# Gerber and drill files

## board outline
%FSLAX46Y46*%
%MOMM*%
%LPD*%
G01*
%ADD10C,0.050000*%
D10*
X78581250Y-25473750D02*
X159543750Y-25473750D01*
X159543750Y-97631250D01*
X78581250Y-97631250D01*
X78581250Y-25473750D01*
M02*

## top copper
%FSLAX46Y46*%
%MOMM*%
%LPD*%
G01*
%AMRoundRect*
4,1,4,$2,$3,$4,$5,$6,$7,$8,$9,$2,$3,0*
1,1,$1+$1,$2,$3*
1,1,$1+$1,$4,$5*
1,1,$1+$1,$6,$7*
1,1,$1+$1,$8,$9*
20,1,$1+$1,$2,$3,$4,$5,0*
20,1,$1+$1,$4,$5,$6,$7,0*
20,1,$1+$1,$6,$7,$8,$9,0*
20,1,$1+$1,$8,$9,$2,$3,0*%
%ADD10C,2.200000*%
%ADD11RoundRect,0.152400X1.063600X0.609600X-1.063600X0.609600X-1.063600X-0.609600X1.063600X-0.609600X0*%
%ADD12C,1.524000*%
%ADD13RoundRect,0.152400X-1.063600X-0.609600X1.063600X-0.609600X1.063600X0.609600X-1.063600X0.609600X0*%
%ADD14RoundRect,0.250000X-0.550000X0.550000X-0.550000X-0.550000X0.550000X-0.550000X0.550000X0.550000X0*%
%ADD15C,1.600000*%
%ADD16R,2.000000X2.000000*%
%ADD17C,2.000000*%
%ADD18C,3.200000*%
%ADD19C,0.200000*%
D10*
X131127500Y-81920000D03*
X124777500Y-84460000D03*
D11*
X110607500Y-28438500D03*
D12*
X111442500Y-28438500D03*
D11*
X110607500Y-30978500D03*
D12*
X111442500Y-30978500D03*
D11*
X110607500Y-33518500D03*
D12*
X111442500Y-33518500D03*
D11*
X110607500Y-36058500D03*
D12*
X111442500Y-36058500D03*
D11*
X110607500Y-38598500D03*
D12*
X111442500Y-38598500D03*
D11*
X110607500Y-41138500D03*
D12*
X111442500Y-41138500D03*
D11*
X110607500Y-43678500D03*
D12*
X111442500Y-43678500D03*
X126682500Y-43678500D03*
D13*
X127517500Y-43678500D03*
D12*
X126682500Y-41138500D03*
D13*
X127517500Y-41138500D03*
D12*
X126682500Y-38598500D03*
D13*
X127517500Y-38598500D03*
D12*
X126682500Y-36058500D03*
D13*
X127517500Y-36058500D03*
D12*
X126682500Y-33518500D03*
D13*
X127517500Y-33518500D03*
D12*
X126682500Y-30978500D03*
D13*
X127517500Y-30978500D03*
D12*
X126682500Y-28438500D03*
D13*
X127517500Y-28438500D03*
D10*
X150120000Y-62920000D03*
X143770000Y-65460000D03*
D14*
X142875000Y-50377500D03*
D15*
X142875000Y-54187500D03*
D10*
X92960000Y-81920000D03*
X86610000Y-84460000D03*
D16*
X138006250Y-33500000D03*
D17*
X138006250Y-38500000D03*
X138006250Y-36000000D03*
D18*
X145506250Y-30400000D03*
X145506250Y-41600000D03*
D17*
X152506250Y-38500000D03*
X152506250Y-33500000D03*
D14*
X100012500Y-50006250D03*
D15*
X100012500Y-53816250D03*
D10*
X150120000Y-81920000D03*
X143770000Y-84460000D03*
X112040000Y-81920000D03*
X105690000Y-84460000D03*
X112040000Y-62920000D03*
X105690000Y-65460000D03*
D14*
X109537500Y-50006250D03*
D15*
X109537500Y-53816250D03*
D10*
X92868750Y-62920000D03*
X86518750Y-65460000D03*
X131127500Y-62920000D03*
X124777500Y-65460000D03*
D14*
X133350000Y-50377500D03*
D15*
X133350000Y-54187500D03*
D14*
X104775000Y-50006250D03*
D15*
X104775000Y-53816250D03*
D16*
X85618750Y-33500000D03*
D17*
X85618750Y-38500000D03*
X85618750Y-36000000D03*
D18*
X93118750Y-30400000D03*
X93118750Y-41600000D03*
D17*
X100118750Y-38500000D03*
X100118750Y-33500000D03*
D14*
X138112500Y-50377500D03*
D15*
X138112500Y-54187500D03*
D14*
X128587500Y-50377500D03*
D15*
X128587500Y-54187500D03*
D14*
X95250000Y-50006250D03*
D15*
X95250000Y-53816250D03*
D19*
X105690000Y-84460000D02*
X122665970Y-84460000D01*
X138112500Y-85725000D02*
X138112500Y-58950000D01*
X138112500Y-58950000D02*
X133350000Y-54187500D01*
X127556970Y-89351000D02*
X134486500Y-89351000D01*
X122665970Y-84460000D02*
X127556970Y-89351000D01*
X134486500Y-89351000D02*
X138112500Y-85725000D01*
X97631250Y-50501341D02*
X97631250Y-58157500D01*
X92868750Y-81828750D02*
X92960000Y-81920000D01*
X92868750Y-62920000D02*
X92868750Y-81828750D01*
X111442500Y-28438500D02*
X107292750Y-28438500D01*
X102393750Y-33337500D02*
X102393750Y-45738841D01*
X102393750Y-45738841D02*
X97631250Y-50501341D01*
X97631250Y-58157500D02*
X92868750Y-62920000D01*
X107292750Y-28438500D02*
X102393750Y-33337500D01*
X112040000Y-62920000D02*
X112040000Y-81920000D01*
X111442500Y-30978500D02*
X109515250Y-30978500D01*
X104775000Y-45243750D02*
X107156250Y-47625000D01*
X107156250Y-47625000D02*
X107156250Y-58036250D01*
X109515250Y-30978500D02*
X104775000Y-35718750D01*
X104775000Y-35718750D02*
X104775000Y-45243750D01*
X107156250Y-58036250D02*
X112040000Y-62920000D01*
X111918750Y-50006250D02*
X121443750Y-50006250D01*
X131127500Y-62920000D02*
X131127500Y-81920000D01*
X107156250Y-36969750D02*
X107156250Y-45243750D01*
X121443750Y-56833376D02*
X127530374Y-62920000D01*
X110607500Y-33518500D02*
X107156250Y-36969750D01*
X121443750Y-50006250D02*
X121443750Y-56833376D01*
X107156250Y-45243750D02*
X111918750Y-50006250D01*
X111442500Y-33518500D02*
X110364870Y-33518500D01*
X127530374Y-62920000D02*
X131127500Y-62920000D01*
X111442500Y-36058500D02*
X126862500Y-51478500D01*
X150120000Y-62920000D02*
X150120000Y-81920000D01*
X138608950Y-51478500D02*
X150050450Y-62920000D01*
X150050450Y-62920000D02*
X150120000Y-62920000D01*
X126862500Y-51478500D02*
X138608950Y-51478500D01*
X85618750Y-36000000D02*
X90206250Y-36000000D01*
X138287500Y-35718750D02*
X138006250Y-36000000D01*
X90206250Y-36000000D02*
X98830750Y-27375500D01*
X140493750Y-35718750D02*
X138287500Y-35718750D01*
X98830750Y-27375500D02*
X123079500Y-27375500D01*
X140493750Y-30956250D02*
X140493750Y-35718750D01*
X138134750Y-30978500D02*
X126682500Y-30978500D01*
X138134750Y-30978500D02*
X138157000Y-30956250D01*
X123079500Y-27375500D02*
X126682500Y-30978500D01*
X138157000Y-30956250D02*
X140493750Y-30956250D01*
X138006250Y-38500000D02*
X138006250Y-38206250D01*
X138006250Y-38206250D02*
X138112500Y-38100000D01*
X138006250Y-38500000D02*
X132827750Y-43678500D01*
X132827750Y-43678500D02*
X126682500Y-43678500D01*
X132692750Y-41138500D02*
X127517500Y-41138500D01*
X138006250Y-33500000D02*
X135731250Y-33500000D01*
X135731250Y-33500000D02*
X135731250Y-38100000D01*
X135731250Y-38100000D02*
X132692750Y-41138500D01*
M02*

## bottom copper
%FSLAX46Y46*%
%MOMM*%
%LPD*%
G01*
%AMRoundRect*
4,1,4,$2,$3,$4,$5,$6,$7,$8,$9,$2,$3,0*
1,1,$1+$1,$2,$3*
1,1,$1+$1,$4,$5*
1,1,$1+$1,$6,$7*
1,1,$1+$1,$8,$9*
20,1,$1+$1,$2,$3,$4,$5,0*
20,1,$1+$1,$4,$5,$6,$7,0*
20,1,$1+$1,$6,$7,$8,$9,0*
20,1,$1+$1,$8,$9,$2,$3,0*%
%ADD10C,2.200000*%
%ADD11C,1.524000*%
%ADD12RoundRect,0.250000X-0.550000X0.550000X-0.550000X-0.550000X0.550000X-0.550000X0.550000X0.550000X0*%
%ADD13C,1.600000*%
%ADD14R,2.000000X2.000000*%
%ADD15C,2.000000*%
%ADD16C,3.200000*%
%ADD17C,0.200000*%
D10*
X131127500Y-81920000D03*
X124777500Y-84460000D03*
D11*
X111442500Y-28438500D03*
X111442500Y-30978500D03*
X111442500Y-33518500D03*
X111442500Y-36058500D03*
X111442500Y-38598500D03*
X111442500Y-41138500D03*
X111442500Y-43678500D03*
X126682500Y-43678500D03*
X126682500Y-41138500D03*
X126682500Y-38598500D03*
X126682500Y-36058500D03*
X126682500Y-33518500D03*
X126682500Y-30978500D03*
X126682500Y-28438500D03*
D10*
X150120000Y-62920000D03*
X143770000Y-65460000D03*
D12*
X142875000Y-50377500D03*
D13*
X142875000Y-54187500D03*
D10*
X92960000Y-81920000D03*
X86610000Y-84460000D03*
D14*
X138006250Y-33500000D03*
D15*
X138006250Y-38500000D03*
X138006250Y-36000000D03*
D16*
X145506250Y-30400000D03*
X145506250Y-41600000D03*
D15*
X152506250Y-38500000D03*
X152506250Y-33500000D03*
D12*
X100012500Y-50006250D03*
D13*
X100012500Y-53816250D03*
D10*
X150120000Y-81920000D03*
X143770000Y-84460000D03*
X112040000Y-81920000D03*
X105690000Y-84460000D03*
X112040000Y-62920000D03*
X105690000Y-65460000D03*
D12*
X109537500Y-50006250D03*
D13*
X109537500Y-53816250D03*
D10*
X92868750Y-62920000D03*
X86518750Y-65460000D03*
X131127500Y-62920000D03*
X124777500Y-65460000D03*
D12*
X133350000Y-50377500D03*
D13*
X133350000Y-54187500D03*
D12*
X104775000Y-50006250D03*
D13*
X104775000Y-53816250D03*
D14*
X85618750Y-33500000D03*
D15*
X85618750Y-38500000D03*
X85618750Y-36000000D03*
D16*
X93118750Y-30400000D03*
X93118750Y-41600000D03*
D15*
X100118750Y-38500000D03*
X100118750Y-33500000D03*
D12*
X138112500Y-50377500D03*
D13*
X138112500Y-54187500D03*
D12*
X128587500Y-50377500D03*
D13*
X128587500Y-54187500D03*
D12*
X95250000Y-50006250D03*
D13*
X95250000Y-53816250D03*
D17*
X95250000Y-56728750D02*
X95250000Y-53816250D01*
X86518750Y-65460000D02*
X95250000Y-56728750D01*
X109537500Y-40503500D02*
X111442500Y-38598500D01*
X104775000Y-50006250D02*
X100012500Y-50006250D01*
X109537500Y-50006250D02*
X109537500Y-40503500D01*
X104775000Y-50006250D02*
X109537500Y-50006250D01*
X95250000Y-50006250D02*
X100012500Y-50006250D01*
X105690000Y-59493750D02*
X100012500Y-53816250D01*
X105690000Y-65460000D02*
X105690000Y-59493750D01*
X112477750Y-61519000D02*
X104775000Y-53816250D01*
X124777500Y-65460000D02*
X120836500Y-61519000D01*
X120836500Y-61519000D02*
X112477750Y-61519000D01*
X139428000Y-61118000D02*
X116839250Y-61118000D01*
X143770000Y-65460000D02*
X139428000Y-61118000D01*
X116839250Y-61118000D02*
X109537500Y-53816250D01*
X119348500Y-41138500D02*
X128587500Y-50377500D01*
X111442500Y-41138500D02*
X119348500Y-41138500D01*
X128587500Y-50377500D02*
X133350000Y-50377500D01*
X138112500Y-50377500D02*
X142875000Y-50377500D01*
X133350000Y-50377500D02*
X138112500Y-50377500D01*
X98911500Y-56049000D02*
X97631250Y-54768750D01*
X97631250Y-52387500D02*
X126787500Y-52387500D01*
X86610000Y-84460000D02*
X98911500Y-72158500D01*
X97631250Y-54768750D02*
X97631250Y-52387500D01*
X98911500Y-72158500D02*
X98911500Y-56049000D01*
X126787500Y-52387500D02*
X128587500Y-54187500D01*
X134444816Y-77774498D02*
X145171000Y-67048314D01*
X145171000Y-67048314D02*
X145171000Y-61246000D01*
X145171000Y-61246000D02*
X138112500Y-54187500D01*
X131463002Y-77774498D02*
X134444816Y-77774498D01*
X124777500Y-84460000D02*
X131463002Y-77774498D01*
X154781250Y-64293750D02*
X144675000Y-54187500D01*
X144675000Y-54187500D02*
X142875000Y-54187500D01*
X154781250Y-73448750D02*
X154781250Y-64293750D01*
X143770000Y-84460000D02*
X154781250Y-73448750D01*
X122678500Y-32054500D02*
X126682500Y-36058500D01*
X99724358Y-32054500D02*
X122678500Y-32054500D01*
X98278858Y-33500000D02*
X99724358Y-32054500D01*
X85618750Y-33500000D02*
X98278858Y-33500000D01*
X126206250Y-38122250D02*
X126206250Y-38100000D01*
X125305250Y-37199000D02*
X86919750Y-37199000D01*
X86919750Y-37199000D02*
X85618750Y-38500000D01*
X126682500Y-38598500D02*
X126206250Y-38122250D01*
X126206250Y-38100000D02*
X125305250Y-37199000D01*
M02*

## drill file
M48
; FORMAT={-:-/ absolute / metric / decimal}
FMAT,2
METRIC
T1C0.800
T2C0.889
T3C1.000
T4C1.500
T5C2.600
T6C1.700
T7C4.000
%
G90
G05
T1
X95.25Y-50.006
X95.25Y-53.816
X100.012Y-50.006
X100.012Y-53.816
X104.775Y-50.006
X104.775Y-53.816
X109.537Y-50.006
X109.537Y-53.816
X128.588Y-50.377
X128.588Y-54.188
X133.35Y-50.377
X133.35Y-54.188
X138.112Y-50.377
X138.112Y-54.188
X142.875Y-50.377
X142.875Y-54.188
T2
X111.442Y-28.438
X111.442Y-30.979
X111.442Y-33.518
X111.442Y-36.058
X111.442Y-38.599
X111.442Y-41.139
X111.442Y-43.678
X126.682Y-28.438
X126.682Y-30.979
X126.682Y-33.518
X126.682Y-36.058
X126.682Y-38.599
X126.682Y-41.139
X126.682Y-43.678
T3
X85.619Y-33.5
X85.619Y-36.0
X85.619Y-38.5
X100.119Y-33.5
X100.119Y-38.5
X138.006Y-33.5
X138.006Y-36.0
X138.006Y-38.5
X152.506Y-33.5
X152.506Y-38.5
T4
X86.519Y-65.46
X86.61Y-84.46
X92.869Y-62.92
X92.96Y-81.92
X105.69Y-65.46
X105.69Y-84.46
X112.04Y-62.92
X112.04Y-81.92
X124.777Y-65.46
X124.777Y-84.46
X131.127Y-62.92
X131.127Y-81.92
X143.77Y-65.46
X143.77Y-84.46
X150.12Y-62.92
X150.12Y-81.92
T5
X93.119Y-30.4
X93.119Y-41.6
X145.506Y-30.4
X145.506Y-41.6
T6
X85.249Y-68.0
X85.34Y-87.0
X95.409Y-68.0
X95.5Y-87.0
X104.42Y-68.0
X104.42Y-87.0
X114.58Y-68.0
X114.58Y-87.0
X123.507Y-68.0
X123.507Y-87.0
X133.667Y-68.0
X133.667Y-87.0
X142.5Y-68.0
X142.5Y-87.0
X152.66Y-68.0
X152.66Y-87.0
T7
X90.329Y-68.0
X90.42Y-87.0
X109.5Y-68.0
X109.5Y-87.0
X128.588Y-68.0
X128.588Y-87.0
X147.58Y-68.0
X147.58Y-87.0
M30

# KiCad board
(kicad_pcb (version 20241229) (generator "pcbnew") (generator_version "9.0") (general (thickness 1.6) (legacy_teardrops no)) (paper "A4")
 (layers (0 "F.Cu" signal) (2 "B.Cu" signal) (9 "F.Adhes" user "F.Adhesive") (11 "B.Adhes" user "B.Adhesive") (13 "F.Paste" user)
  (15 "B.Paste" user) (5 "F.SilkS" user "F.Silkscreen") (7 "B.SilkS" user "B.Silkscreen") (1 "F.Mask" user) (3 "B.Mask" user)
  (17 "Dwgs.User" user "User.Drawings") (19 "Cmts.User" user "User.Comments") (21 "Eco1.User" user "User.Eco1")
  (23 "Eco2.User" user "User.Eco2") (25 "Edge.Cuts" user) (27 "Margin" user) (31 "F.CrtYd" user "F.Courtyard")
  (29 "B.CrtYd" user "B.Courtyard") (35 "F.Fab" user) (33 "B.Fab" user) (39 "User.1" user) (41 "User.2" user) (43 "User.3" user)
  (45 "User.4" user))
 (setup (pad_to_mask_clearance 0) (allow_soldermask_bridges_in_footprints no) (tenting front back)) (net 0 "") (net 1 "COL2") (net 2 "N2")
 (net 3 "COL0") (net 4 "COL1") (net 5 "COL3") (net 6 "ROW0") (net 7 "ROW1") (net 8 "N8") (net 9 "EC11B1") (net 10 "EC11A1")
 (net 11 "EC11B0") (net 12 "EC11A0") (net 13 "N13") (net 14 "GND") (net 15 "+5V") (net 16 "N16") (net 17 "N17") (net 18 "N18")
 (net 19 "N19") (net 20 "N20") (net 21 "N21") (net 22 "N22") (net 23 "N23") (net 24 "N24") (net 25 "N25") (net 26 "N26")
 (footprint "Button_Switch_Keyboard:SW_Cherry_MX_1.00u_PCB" (layer "F.Cu") (at 131.1275 81.92)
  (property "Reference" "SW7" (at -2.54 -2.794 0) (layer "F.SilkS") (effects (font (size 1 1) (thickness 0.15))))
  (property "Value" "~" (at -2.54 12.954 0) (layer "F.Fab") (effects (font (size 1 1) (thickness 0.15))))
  (pad "" np_thru_hole circle (at -7.62 5.08) (size 1.7 1.7) (drill 1.7) (layers "*.Cu" "*.Mask"))
  (pad "" np_thru_hole circle (at -2.54 5.08) (size 4 4) (drill 4) (layers "*.Cu" "*.Mask"))
  (pad "" np_thru_hole circle (at 2.54 5.08) (size 1.7 1.7) (drill 1.7) (layers "*.Cu" "*.Mask"))
  (pad "1" thru_hole circle (at 0 0) (size 2.2 2.2) (drill 1.5) (layers "*.Cu" "*.Mask") (remove_unused_layers no) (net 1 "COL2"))
  (pad "2" thru_hole circle (at -6.35 2.54) (size 2.2 2.2) (drill 1.5) (layers "*.Cu" "*.Mask") (remove_unused_layers no) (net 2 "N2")))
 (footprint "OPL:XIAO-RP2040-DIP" (layer "F.Cu") (at 119.0625 36.0585)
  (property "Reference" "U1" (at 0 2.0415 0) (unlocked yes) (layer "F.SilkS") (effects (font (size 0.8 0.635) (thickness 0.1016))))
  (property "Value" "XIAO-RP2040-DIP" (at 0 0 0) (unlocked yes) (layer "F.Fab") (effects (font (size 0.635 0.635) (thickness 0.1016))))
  (pad "1" smd roundrect (at -8.455 -7.62 180) (size 2.432 1.524) (layers "F.Cu" "F.Mask") (roundrect_rratio 0.1) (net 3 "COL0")
   (thermal_bridge_angle 45))
  (pad "1" thru_hole circle (at -7.62 -7.62 180) (size 1.524 1.524) (drill 0.889) (layers "*.Cu" "*.Mask") (remove_unused_layers no)
   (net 3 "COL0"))
  (pad "2" smd roundrect (at -8.455 -5.08 180) (size 2.432 1.524) (layers "F.Cu" "F.Mask") (roundrect_rratio 0.1) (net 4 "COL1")
   (thermal_bridge_angle 45))
  (pad "2" thru_hole circle (at -7.62 -5.08 180) (size 1.524 1.524) (drill 0.889) (layers "*.Cu" "*.Mask") (remove_unused_layers no)
   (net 4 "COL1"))
  (pad "3" smd roundrect (at -8.455 -2.54 180) (size 2.432 1.524) (layers "F.Cu" "F.Mask") (roundrect_rratio 0.1) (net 1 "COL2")
   (thermal_bridge_angle 45))
  (pad "3" thru_hole circle (at -7.62 -2.54 180) (size 1.524 1.524) (drill 0.889) (layers "*.Cu" "*.Mask") (remove_unused_layers no)
   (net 1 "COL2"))
  (pad "4" smd roundrect (at -8.455 0 180) (size 2.432 1.524) (layers "F.Cu" "F.Mask") (roundrect_rratio 0.1) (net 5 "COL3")
   (thermal_bridge_angle 45))
  (pad "4" thru_hole circle (at -7.62 0 180) (size 1.524 1.524) (drill 0.889) (layers "*.Cu" "*.Mask") (remove_unused_layers no)
   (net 5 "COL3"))
  (pad "5" smd roundrect (at -8.455 2.54 180) (size 2.432 1.524) (layers "F.Cu" "F.Mask") (roundrect_rratio 0.1) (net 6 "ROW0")
   (thermal_bridge_angle 45))
  (pad "5" thru_hole circle (at -7.62 2.54 180) (size 1.524 1.524) (drill 0.889) (layers "*.Cu" "*.Mask") (remove_unused_layers no)
   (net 6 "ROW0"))
  (pad "6" smd roundrect (at -8.455 5.08 180) (size 2.432 1.524) (layers "F.Cu" "F.Mask") (roundrect_rratio 0.1) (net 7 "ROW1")
   (thermal_bridge_angle 45))
  (pad "6" thru_hole circle (at -7.62 5.08 180) (size 1.524 1.524) (drill 0.889) (layers "*.Cu" "*.Mask") (remove_unused_layers no)
   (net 7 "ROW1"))
  (pad "7" smd roundrect (at -8.455 7.62 180) (size 2.432 1.524) (layers "F.Cu" "F.Mask") (roundrect_rratio 0.1) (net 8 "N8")
   (thermal_bridge_angle 45))
  (pad "7" thru_hole circle (at -7.62 7.62 180) (size 1.524 1.524) (drill 0.889) (layers "*.Cu" "*.Mask") (remove_unused_layers no)
   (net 8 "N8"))
  (pad "8" thru_hole circle (at 7.62 7.62) (size 1.524 1.524) (drill 0.889) (layers "*.Cu" "*.Mask") (remove_unused_layers no)
   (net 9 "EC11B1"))
  (pad "8" smd roundrect (at 8.455 7.62) (size 2.432 1.524) (layers "F.Cu" "F.Mask") (roundrect_rratio 0.1) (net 9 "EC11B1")
   (thermal_bridge_angle 45))
  (pad "9" thru_hole circle (at 7.62 5.08) (size 1.524 1.524) (drill 0.889) (layers "*.Cu" "*.Mask") (remove_unused_layers no)
   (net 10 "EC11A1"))
  (pad "9" smd roundrect (at 8.455 5.08) (size 2.432 1.524) (layers "F.Cu" "F.Mask") (roundrect_rratio 0.1) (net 10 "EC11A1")
   (thermal_bridge_angle 45))
  (pad "10" thru_hole circle (at 7.62 2.54) (size 1.524 1.524) (drill 0.889) (layers "*.Cu" "*.Mask") (remove_unused_layers no)
   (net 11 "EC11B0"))
  (pad "10" smd roundrect (at 8.455 2.54) (size 2.432 1.524) (layers "F.Cu" "F.Mask") (roundrect_rratio 0.1) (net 11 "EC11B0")
   (thermal_bridge_angle 45))
  (pad "11" thru_hole circle (at 7.62 0) (size 1.524 1.524) (drill 0.889) (layers "*.Cu" "*.Mask") (remove_unused_layers no)
   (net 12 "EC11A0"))
  (pad "11" smd roundrect (at 8.455 0) (size 2.432 1.524) (layers "F.Cu" "F.Mask") (roundrect_rratio 0.1) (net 12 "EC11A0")
   (thermal_bridge_angle 45))
  (pad "12" thru_hole circle (at 7.62 -2.54) (size 1.524 1.524) (drill 0.889) (layers "*.Cu" "*.Mask") (remove_unused_layers no)
   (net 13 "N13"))
  (pad "12" smd roundrect (at 8.455 -2.54) (size 2.432 1.524) (layers "F.Cu" "F.Mask") (roundrect_rratio 0.1) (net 13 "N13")
   (thermal_bridge_angle 45))
  (pad "13" thru_hole circle (at 7.62 -5.08) (size 1.524 1.524) (drill 0.889) (layers "*.Cu" "*.Mask") (remove_unused_layers no)
   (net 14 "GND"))
  (pad "13" smd roundrect (at 8.455 -5.08) (size 2.432 1.524) (layers "F.Cu" "F.Mask") (roundrect_rratio 0.1) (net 14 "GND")
   (thermal_bridge_angle 45))
  (pad "14" thru_hole circle (at 7.62 -7.62) (size 1.524 1.524) (drill 0.889) (layers "*.Cu" "*.Mask") (remove_unused_layers no)
   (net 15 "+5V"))
  (pad "14" smd roundrect (at 8.455 -7.62) (size 2.432 1.524) (layers "F.Cu" "F.Mask") (roundrect_rratio 0.1) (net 15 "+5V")
   (thermal_bridge_angle 45)))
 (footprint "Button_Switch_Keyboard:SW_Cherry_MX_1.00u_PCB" (layer "F.Cu") (at 150.12 62.92)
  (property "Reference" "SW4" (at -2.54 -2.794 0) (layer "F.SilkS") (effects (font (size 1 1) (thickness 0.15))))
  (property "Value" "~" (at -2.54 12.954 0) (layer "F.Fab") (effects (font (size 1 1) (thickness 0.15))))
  (pad "" np_thru_hole circle (at -7.62 5.08) (size 1.7 1.7) (drill 1.7) (layers "*.Cu" "*.Mask"))
  (pad "" np_thru_hole circle (at -2.54 5.08) (size 4 4) (drill 4) (layers "*.Cu" "*.Mask"))
  (pad "" np_thru_hole circle (at 2.54 5.08) (size 1.7 1.7) (drill 1.7) (layers "*.Cu" "*.Mask"))
  (pad "1" thru_hole circle (at 0 0) (size 2.2 2.2) (drill 1.5) (layers "*.Cu" "*.Mask") (remove_unused_layers no) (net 5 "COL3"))
  (pad "2" thru_hole circle (at -6.35 2.54) (size 2.2 2.2) (drill 1.5) (layers "*.Cu" "*.Mask") (remove_unused_layers no) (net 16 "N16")))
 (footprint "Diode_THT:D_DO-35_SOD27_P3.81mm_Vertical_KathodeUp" (layer "F.Cu") (at 142.875 50.3775 -90)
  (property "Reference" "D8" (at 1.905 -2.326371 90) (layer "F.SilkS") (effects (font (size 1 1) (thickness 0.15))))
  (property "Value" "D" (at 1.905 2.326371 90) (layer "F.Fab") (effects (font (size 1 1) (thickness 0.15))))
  (pad "1" thru_hole roundrect (at 0 0 270) (size 1.6 1.6) (drill 0.8) (layers "*.Cu" "*.Mask") (remove_unused_layers no)
   (roundrect_rratio 0.15625) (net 7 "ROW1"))
  (pad "2" thru_hole circle (at 3.81 0 270) (size 1.6 1.6) (drill 0.8) (layers "*.Cu" "*.Mask") (remove_unused_layers no) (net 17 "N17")))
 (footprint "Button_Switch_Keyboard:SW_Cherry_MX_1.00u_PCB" (layer "F.Cu") (at 92.96 81.92)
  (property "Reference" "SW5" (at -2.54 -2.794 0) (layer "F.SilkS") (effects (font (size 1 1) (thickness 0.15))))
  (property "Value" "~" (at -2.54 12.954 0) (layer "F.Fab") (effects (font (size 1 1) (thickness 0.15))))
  (pad "" np_thru_hole circle (at -7.62 5.08) (size 1.7 1.7) (drill 1.7) (layers "*.Cu" "*.Mask"))
  (pad "" np_thru_hole circle (at -2.54 5.08) (size 4 4) (drill 4) (layers "*.Cu" "*.Mask"))
  (pad "" np_thru_hole circle (at 2.54 5.08) (size 1.7 1.7) (drill 1.7) (layers "*.Cu" "*.Mask"))
  (pad "1" thru_hole circle (at 0 0) (size 2.2 2.2) (drill 1.5) (layers "*.Cu" "*.Mask") (remove_unused_layers no) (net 3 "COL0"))
  (pad "2" thru_hole circle (at -6.35 2.54) (size 2.2 2.2) (drill 1.5) (layers "*.Cu" "*.Mask") (remove_unused_layers no) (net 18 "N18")))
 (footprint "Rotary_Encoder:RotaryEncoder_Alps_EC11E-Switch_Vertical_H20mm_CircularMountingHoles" (layer "F.Cu") (at 138.00625 33.5)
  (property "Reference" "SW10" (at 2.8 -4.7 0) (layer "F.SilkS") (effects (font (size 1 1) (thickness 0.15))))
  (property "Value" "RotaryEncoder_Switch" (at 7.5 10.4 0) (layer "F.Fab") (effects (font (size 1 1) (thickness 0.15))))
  (pad "A" thru_hole rect (at 0 0) (size 2 2) (drill 1) (layers "*.Cu" "*.Mask") (remove_unused_layers no) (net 10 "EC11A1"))
  (pad "B" thru_hole circle (at 0 5) (size 2 2) (drill 1) (layers "*.Cu" "*.Mask") (remove_unused_layers no) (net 9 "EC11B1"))
  (pad "C" thru_hole circle (at 0 2.5) (size 2 2) (drill 1) (layers "*.Cu" "*.Mask") (remove_unused_layers no) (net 14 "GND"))
  (pad "MP" thru_hole circle (at 7.5 -3.1) (size 3.2 3.2) (drill 2.6) (layers "*.Cu" "*.Mask") (remove_unused_layers no))
  (pad "MP" thru_hole circle (at 7.5 8.1) (size 3.2 3.2) (drill 2.6) (layers "*.Cu" "*.Mask") (remove_unused_layers no))
  (pad "S1" thru_hole circle (at 14.5 5) (size 2 2) (drill 1) (layers "*.Cu" "*.Mask") (remove_unused_layers no) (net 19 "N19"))
  (pad "S2" thru_hole circle (at 14.5 0) (size 2 2) (drill 1) (layers "*.Cu" "*.Mask") (remove_unused_layers no) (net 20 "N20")))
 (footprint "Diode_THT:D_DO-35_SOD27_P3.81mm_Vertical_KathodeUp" (layer "F.Cu") (at 100.0125 50.00625 -90)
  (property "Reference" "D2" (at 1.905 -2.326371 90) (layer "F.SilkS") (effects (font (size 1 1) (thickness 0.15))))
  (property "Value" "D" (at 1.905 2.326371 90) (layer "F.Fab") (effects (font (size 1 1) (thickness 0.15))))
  (pad "1" thru_hole roundrect (at 0 0 270) (size 1.6 1.6) (drill 0.8) (layers "*.Cu" "*.Mask") (remove_unused_layers no)
   (roundrect_rratio 0.15625) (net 6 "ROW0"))
  (pad "2" thru_hole circle (at 3.81 0 270) (size 1.6 1.6) (drill 0.8) (layers "*.Cu" "*.Mask") (remove_unused_layers no) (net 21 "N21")))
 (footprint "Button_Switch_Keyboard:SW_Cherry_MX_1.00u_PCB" (layer "F.Cu") (at 150.12 81.92)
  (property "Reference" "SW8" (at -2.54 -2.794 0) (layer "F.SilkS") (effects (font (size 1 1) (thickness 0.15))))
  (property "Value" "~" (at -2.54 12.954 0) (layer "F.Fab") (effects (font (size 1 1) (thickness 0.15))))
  (pad "" np_thru_hole circle (at -7.62 5.08) (size 1.7 1.7) (drill 1.7) (layers "*.Cu" "*.Mask"))
  (pad "" np_thru_hole circle (at -2.54 5.08) (size 4 4) (drill 4) (layers "*.Cu" "*.Mask"))
  (pad "" np_thru_hole circle (at 2.54 5.08) (size 1.7 1.7) (drill 1.7) (layers "*.Cu" "*.Mask"))
  (pad "1" thru_hole circle (at 0 0) (size 2.2 2.2) (drill 1.5) (layers "*.Cu" "*.Mask") (remove_unused_layers no) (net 5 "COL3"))
  (pad "2" thru_hole circle (at -6.35 2.54) (size 2.2 2.2) (drill 1.5) (layers "*.Cu" "*.Mask") (remove_unused_layers no) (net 17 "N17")))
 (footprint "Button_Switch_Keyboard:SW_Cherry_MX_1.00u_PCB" (layer "F.Cu") (at 112.04 81.92)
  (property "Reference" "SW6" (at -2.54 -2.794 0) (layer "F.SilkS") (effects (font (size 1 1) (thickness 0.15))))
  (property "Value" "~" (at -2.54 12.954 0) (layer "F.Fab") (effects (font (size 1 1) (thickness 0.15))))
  (pad "" np_thru_hole circle (at -7.62 5.08) (size 1.7 1.7) (drill 1.7) (layers "*.Cu" "*.Mask"))
  (pad "" np_thru_hole circle (at -2.54 5.08) (size 4 4) (drill 4) (layers "*.Cu" "*.Mask"))
  (pad "" np_thru_hole circle (at 2.54 5.08) (size 1.7 1.7) (drill 1.7) (layers "*.Cu" "*.Mask"))
  (pad "1" thru_hole circle (at 0 0) (size 2.2 2.2) (drill 1.5) (layers "*.Cu" "*.Mask") (remove_unused_layers no) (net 4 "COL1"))
  (pad "2" thru_hole circle (at -6.35 2.54) (size 2.2 2.2) (drill 1.5) (layers "*.Cu" "*.Mask") (remove_unused_layers no) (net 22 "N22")))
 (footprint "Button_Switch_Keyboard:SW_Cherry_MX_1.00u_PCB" (layer "F.Cu") (at 112.04 62.92)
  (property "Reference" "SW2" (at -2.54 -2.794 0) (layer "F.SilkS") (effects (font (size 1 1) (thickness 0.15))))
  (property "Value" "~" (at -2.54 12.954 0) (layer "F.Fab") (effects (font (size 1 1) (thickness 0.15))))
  (pad "" np_thru_hole circle (at -7.62 5.08) (size 1.7 1.7) (drill 1.7) (layers "*.Cu" "*.Mask"))
  (pad "" np_thru_hole circle (at -2.54 5.08) (size 4 4) (drill 4) (layers "*.Cu" "*.Mask"))
  (pad "" np_thru_hole circle (at 2.54 5.08) (size 1.7 1.7) (drill 1.7) (layers "*.Cu" "*.Mask"))
  (pad "1" thru_hole circle (at 0 0) (size 2.2 2.2) (drill 1.5) (layers "*.Cu" "*.Mask") (remove_unused_layers no) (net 4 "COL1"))
  (pad "2" thru_hole circle (at -6.35 2.54) (size 2.2 2.2) (drill 1.5) (layers "*.Cu" "*.Mask") (remove_unused_layers no) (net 21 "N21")))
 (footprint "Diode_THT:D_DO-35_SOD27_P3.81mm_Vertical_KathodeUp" (layer "F.Cu") (at 109.5375 50.00625 -90)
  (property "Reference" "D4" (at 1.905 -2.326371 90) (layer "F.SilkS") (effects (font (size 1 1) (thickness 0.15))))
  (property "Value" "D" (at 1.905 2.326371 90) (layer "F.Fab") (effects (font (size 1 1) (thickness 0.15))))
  (pad "1" thru_hole roundrect (at 0 0 270) (size 1.6 1.6) (drill 0.8) (layers "*.Cu" "*.Mask") (remove_unused_layers no)
   (roundrect_rratio 0.15625) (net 6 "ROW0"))
  (pad "2" thru_hole circle (at 3.81 0 270) (size 1.6 1.6) (drill 0.8) (layers "*.Cu" "*.Mask") (remove_unused_layers no) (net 16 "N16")))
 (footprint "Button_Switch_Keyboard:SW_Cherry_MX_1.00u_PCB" (layer "F.Cu") (at 92.86875 62.92)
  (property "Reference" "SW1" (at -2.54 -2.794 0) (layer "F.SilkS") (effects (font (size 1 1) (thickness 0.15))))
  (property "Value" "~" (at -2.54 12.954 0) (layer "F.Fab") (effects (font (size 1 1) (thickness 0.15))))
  (pad "" np_thru_hole circle (at -7.62 5.08) (size 1.7 1.7) (drill 1.7) (layers "*.Cu" "*.Mask"))
  (pad "" np_thru_hole circle (at -2.54 5.08) (size 4 4) (drill 4) (layers "*.Cu" "*.Mask"))
  (pad "" np_thru_hole circle (at 2.54 5.08) (size 1.7 1.7) (drill 1.7) (layers "*.Cu" "*.Mask"))
  (pad "1" thru_hole circle (at 0 0) (size 2.2 2.2) (drill 1.5) (layers "*.Cu" "*.Mask") (remove_unused_layers no) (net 3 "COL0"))
  (pad "2" thru_hole circle (at -6.35 2.54) (size 2.2 2.2) (drill 1.5) (layers "*.Cu" "*.Mask") (remove_unused_layers no) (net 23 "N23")))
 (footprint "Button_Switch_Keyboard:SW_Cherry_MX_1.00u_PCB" (layer "F.Cu") (at 131.1275 62.92)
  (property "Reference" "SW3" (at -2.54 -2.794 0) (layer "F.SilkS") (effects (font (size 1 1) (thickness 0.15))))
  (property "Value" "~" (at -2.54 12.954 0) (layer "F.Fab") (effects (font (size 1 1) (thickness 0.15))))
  (pad "" np_thru_hole circle (at -7.62 5.08) (size 1.7 1.7) (drill 1.7) (layers "*.Cu" "*.Mask"))
  (pad "" np_thru_hole circle (at -2.54 5.08) (size 4 4) (drill 4) (layers "*.Cu" "*.Mask"))
  (pad "" np_thru_hole circle (at 2.54 5.08) (size 1.7 1.7) (drill 1.7) (layers "*.Cu" "*.Mask"))
  (pad "1" thru_hole circle (at 0 0) (size 2.2 2.2) (drill 1.5) (layers "*.Cu" "*.Mask") (remove_unused_layers no) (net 1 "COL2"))
  (pad "2" thru_hole circle (at -6.35 2.54) (size 2.2 2.2) (drill 1.5) (layers "*.Cu" "*.Mask") (remove_unused_layers no) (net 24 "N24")))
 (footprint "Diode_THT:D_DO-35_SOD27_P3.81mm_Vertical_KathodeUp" (layer "F.Cu") (at 133.35 50.3775 -90)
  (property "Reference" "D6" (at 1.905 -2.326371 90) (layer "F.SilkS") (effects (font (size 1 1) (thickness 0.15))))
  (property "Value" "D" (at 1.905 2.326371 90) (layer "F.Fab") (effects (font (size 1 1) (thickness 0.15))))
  (pad "1" thru_hole roundrect (at 0 0 270) (size 1.6 1.6) (drill 0.8) (layers "*.Cu" "*.Mask") (remove_unused_layers no)
   (roundrect_rratio 0.15625) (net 7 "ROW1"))
  (pad "2" thru_hole circle (at 3.81 0 270) (size 1.6 1.6) (drill 0.8) (layers "*.Cu" "*.Mask") (remove_unused_layers no) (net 22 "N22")))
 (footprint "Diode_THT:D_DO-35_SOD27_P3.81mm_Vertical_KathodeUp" (layer "F.Cu") (at 104.775 50.00625 -90)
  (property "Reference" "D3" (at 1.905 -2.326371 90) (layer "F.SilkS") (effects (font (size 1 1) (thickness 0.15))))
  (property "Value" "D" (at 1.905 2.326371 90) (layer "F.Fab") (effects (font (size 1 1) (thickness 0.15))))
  (pad "1" thru_hole roundrect (at 0 0 270) (size 1.6 1.6) (drill 0.8) (layers "*.Cu" "*.Mask") (remove_unused_layers no)
   (roundrect_rratio 0.15625) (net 6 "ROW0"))
  (pad "2" thru_hole circle (at 3.81 0 270) (size 1.6 1.6) (drill 0.8) (layers "*.Cu" "*.Mask") (remove_unused_layers no) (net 24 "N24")))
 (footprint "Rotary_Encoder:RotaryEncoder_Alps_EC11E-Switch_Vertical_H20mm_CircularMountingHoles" (layer "F.Cu") (at 85.61875 33.5)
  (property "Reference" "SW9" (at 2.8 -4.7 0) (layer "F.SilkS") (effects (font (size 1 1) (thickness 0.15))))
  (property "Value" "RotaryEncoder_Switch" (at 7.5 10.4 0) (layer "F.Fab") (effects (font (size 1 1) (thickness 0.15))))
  (pad "A" thru_hole rect (at 0 0) (size 2 2) (drill 1) (layers "*.Cu" "*.Mask") (remove_unused_layers no) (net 12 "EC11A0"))
  (pad "B" thru_hole circle (at 0 5) (size 2 2) (drill 1) (layers "*.Cu" "*.Mask") (remove_unused_layers no) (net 11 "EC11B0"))
  (pad "C" thru_hole circle (at 0 2.5) (size 2 2) (drill 1) (layers "*.Cu" "*.Mask") (remove_unused_layers no) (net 14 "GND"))
  (pad "MP" thru_hole circle (at 7.5 -3.1) (size 3.2 3.2) (drill 2.6) (layers "*.Cu" "*.Mask") (remove_unused_layers no))
  (pad "MP" thru_hole circle (at 7.5 8.1) (size 3.2 3.2) (drill 2.6) (layers "*.Cu" "*.Mask") (remove_unused_layers no))
  (pad "S1" thru_hole circle (at 14.5 5) (size 2 2) (drill 1) (layers "*.Cu" "*.Mask") (remove_unused_layers no) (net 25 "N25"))
  (pad "S2" thru_hole circle (at 14.5 0) (size 2 2) (drill 1) (layers "*.Cu" "*.Mask") (remove_unused_layers no) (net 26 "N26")))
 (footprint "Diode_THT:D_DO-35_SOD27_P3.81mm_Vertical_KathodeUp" (layer "F.Cu") (at 138.1125 50.3775 -90)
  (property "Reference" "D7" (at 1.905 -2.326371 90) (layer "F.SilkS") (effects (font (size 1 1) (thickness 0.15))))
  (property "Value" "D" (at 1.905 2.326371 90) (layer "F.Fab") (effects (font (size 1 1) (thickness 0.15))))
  (pad "1" thru_hole roundrect (at 0 0 270) (size 1.6 1.6) (drill 0.8) (layers "*.Cu" "*.Mask") (remove_unused_layers no)
   (roundrect_rratio 0.15625) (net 7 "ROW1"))
  (pad "2" thru_hole circle (at 3.81 0 270) (size 1.6 1.6) (drill 0.8) (layers "*.Cu" "*.Mask") (remove_unused_layers no) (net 2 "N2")))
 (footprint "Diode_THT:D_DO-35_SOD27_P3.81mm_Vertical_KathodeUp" (layer "F.Cu") (at 128.5875 50.3775 -90)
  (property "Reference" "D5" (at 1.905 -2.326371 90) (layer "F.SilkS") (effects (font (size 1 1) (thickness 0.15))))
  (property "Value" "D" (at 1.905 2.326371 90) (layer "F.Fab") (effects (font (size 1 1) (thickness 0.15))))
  (pad "1" thru_hole roundrect (at 0 0 270) (size 1.6 1.6) (drill 0.8) (layers "*.Cu" "*.Mask") (remove_unused_layers no)
   (roundrect_rratio 0.15625) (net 7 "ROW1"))
  (pad "2" thru_hole circle (at 3.81 0 270) (size 1.6 1.6) (drill 0.8) (layers "*.Cu" "*.Mask") (remove_unused_layers no) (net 18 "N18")))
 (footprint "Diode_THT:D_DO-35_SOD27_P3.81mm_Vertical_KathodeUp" (layer "F.Cu") (at 95.25 50.00625 -90)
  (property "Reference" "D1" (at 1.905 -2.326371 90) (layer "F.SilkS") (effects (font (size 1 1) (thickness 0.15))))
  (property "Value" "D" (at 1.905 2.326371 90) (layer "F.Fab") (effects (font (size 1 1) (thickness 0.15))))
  (pad "1" thru_hole roundrect (at 0 0 270) (size 1.6 1.6) (drill 0.8) (layers "*.Cu" "*.Mask") (remove_unused_layers no)
   (roundrect_rratio 0.15625) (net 6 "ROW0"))
  (pad "2" thru_hole circle (at 3.81 0 270) (size 1.6 1.6) (drill 0.8) (layers "*.Cu" "*.Mask") (remove_unused_layers no) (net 23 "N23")))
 (gr_rect (start 78.58125 25.47375) (end 159.54375 97.63125) (stroke (width 0.05) (type default)) (fill no) (layer "Edge.Cuts"))
 (segment (start 95.25 56.72875) (end 95.25 53.81625) (width 0.2) (layer "B.Cu") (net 23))
 (segment (start 86.51875 65.46) (end 95.25 56.72875) (width 0.2) (layer "B.Cu") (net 23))
 (segment (start 109.5375 40.5035) (end 111.4425 38.5985) (width 0.2) (layer "B.Cu") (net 6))
 (segment (start 104.775 50.00625) (end 100.0125 50.00625) (width 0.2) (layer "B.Cu") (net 6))
 (segment (start 109.5375 50.00625) (end 109.5375 40.5035) (width 0.2) (layer "B.Cu") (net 6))
 (segment (start 104.775 50.00625) (end 109.5375 50.00625) (width 0.2) (layer "B.Cu") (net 6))
 (segment (start 95.25 50.00625) (end 100.0125 50.00625) (width 0.2) (layer "B.Cu") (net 6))
 (segment (start 105.69 59.49375) (end 100.0125 53.81625) (width 0.2) (layer "B.Cu") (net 21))
 (segment (start 105.69 65.46) (end 105.69 59.49375) (width 0.2) (layer "B.Cu") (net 21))
 (segment (start 112.47775 61.519) (end 104.775 53.81625) (width 0.2) (layer "B.Cu") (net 24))
 (segment (start 124.7775 65.46) (end 120.8365 61.519) (width 0.2) (layer "B.Cu") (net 24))
 (segment (start 120.8365 61.519) (end 112.47775 61.519) (width 0.2) (layer "B.Cu") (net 24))
 (segment (start 139.428 61.118) (end 116.83925 61.118) (width 0.2) (layer "B.Cu") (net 16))
 (segment (start 143.77 65.46) (end 139.428 61.118) (width 0.2) (layer "B.Cu") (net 16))
 (segment (start 116.83925 61.118) (end 109.5375 53.81625) (width 0.2) (layer "B.Cu") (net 16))
 (segment (start 119.3485 41.1385) (end 128.5875 50.3775) (width 0.2) (layer "B.Cu") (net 7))
 (segment (start 111.4425 41.1385) (end 119.3485 41.1385) (width 0.2) (layer "B.Cu") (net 7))
 (segment (start 128.5875 50.3775) (end 133.35 50.3775) (width 0.2) (layer "B.Cu") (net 7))
 (segment (start 138.1125 50.3775) (end 142.875 50.3775) (width 0.2) (layer "B.Cu") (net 7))
 (segment (start 133.35 50.3775) (end 138.1125 50.3775) (width 0.2) (layer "B.Cu") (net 7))
 (segment (start 98.9115 56.049) (end 97.63125 54.76875) (width 0.2) (layer "B.Cu") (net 18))
 (segment (start 97.63125 52.3875) (end 126.7875 52.3875) (width 0.2) (layer "B.Cu") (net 18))
 (segment (start 86.61 84.46) (end 98.9115 72.1585) (width 0.2) (layer "B.Cu") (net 18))
 (segment (start 97.63125 54.76875) (end 97.63125 52.3875) (width 0.2) (layer "B.Cu") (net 18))
 (segment (start 98.9115 72.1585) (end 98.9115 56.049) (width 0.2) (layer "B.Cu") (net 18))
 (segment (start 126.7875 52.3875) (end 128.5875 54.1875) (width 0.2) (layer "B.Cu") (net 18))
 (segment (start 105.69 84.46) (end 122.66597 84.46) (width 0.2) (layer "F.Cu") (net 22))
 (segment (start 138.1125 85.725) (end 138.1125 58.95) (width 0.2) (layer "F.Cu") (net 22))
 (segment (start 138.1125 58.95) (end 133.35 54.1875) (width 0.2) (layer "F.Cu") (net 22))
 (segment (start 127.55697 89.351) (end 134.4865 89.351) (width 0.2) (layer "F.Cu") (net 22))
 (segment (start 122.66597 84.46) (end 127.55697 89.351) (width 0.2) (layer "F.Cu") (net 22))
 (segment (start 134.4865 89.351) (end 138.1125 85.725) (width 0.2) (layer "F.Cu") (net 22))
 (segment (start 134.444816 77.774498) (end 145.171 67.048314) (width 0.2) (layer "B.Cu") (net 2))
 (segment (start 145.171 67.048314) (end 145.171 61.246) (width 0.2) (layer "B.Cu") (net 2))
 (segment (start 145.171 61.246) (end 138.1125 54.1875) (width 0.2) (layer "B.Cu") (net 2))
 (segment (start 131.463002 77.774498) (end 134.444816 77.774498) (width 0.2) (layer "B.Cu") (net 2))
 (segment (start 124.7775 84.46) (end 131.463002 77.774498) (width 0.2) (layer "B.Cu") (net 2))
 (segment (start 154.78125 64.29375) (end 144.675 54.1875) (width 0.2) (layer "B.Cu") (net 17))
 (segment (start 144.675 54.1875) (end 142.875 54.1875) (width 0.2) (layer "B.Cu") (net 17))
 (segment (start 154.78125 73.44875) (end 154.78125 64.29375) (width 0.2) (layer "B.Cu") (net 17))
 (segment (start 143.77 84.46) (end 154.78125 73.44875) (width 0.2) (layer "B.Cu") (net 17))
 (segment (start 97.63125 50.501341) (end 97.63125 58.1575) (width 0.2) (layer "F.Cu") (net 3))
 (segment (start 92.86875 81.82875) (end 92.96 81.92) (width 0.2) (layer "F.Cu") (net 3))
 (segment (start 92.86875 62.92) (end 92.86875 81.82875) (width 0.2) (layer "F.Cu") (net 3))
 (segment (start 111.4425 28.4385) (end 107.29275 28.4385) (width 0.2) (layer "F.Cu") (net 3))
 (segment (start 102.39375 33.3375) (end 102.39375 45.738841) (width 0.2) (layer "F.Cu") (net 3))
 (segment (start 102.39375 45.738841) (end 97.63125 50.501341) (width 0.2) (layer "F.Cu") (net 3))
 (segment (start 97.63125 58.1575) (end 92.86875 62.92) (width 0.2) (layer "F.Cu") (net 3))
 (segment (start 107.29275 28.4385) (end 102.39375 33.3375) (width 0.2) (layer "F.Cu") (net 3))
 (segment (start 112.04 62.92) (end 112.04 81.92) (width 0.2) (layer "F.Cu") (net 4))
 (segment (start 111.4425 30.9785) (end 109.51525 30.9785) (width 0.2) (layer "F.Cu") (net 4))
 (segment (start 104.775 45.24375) (end 107.15625 47.625) (width 0.2) (layer "F.Cu") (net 4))
 (segment (start 107.15625 47.625) (end 107.15625 58.03625) (width 0.2) (layer "F.Cu") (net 4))
 (segment (start 109.51525 30.9785) (end 104.775 35.71875) (width 0.2) (layer "F.Cu") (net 4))
 (segment (start 104.775 35.71875) (end 104.775 45.24375) (width 0.2) (layer "F.Cu") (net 4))
 (segment (start 107.15625 58.03625) (end 112.04 62.92) (width 0.2) (layer "F.Cu") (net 4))
 (segment (start 111.91875 50.00625) (end 121.44375 50.00625) (width 0.2) (layer "F.Cu") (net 1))
 (segment (start 131.1275 62.92) (end 131.1275 81.92) (width 0.2) (layer "F.Cu") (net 1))
 (segment (start 107.15625 36.96975) (end 107.15625 45.24375) (width 0.2) (layer "F.Cu") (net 1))
 (segment (start 121.44375 56.833376) (end 127.530374 62.92) (width 0.2) (layer "F.Cu") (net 1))
 (segment (start 110.6075 33.5185) (end 107.15625 36.96975) (width 0.2) (layer "F.Cu") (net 1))
 (segment (start 121.44375 50.00625) (end 121.44375 56.833376) (width 0.2) (layer "F.Cu") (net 1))
 (segment (start 107.15625 45.24375) (end 111.91875 50.00625) (width 0.2) (layer "F.Cu") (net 1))
 (segment (start 111.4425 33.5185) (end 110.36487 33.5185) (width 0.2) (layer "F.Cu") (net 1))
 (segment (start 127.530374 62.92) (end 131.1275 62.92) (width 0.2) (layer "F.Cu") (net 1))
 (segment (start 111.4425 36.0585) (end 126.8625 51.4785) (width 0.2) (layer "F.Cu") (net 5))
 (segment (start 150.12 62.92) (end 150.12 81.92) (width 0.2) (layer "F.Cu") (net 5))
 (segment (start 138.60895 51.4785) (end 150.05045 62.92) (width 0.2) (layer "F.Cu") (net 5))
 (segment (start 150.05045 62.92) (end 150.12 62.92) (width 0.2) (layer "F.Cu") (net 5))
 (segment (start 126.8625 51.4785) (end 138.60895 51.4785) (width 0.2) (layer "F.Cu") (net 5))
 (segment (start 122.6785 32.0545) (end 126.6825 36.0585) (width 0.2) (layer "B.Cu") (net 12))
 (segment (start 99.724358 32.0545) (end 122.6785 32.0545) (width 0.2) (layer "B.Cu") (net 12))
 (segment (start 98.278858 33.5) (end 99.724358 32.0545) (width 0.2) (layer "B.Cu") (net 12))
 (segment (start 85.61875 33.5) (end 98.278858 33.5) (width 0.2) (layer "B.Cu") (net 12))
 (segment (start 85.61875 36) (end 90.20625 36) (width 0.2) (layer "F.Cu") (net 14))
 (segment (start 138.2875 35.71875) (end 138.00625 36) (width 0.2) (layer "F.Cu") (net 14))
 (segment (start 90.20625 36) (end 98.83075 27.3755) (width 0.2) (layer "F.Cu") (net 14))
 (segment (start 140.49375 35.71875) (end 138.2875 35.71875) (width 0.2) (layer "F.Cu") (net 14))
 (segment (start 98.83075 27.3755) (end 123.0795 27.3755) (width 0.2) (layer "F.Cu") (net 14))
 (segment (start 140.49375 30.95625) (end 140.49375 35.71875) (width 0.2) (layer "F.Cu") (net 14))
 (segment (start 138.13475 30.9785) (end 126.6825 30.9785) (width 0.2) (layer "F.Cu") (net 14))
 (segment (start 138.13475 30.9785) (end 138.157 30.95625) (width 0.2) (layer "F.Cu") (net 14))
 (segment (start 123.0795 27.3755) (end 126.6825 30.9785) (width 0.2) (layer "F.Cu") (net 14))
 (segment (start 138.157 30.95625) (end 140.49375 30.95625) (width 0.2) (layer "F.Cu") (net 14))
 (segment (start 126.20625 38.12225) (end 126.20625 38.1) (width 0.2) (layer "B.Cu") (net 11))
 (segment (start 125.30525 37.199) (end 86.91975 37.199) (width 0.2) (layer "B.Cu") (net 11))
 (segment (start 86.91975 37.199) (end 85.61875 38.5) (width 0.2) (layer "B.Cu") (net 11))
 (segment (start 126.6825 38.5985) (end 126.20625 38.12225) (width 0.2) (layer "B.Cu") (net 11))
 (segment (start 126.20625 38.1) (end 125.30525 37.199) (width 0.2) (layer "B.Cu") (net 11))
 (segment (start 138.00625 38.5) (end 138.00625 38.20625) (width 0.2) (layer "F.Cu") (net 9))
 (segment (start 138.00625 38.20625) (end 138.1125 38.1) (width 0.2) (layer "F.Cu") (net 9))
 (segment (start 138.00625 38.5) (end 132.82775 43.6785) (width 0.2) (layer "F.Cu") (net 9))
 (segment (start 132.82775 43.6785) (end 126.6825 43.6785) (width 0.2) (layer "F.Cu") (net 9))
 (segment (start 132.69275 41.1385) (end 127.5175 41.1385) (width 0.2) (layer "F.Cu") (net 10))
 (segment (start 138.00625 33.5) (end 135.73125 33.5) (width 0.2) (layer "F.Cu") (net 10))
 (segment (start 135.73125 33.5) (end 135.73125 38.1) (width 0.2) (layer "F.Cu") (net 10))
 (segment (start 135.73125 38.1) (end 132.69275 41.1385) (width 0.2) (layer "F.Cu") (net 10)))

